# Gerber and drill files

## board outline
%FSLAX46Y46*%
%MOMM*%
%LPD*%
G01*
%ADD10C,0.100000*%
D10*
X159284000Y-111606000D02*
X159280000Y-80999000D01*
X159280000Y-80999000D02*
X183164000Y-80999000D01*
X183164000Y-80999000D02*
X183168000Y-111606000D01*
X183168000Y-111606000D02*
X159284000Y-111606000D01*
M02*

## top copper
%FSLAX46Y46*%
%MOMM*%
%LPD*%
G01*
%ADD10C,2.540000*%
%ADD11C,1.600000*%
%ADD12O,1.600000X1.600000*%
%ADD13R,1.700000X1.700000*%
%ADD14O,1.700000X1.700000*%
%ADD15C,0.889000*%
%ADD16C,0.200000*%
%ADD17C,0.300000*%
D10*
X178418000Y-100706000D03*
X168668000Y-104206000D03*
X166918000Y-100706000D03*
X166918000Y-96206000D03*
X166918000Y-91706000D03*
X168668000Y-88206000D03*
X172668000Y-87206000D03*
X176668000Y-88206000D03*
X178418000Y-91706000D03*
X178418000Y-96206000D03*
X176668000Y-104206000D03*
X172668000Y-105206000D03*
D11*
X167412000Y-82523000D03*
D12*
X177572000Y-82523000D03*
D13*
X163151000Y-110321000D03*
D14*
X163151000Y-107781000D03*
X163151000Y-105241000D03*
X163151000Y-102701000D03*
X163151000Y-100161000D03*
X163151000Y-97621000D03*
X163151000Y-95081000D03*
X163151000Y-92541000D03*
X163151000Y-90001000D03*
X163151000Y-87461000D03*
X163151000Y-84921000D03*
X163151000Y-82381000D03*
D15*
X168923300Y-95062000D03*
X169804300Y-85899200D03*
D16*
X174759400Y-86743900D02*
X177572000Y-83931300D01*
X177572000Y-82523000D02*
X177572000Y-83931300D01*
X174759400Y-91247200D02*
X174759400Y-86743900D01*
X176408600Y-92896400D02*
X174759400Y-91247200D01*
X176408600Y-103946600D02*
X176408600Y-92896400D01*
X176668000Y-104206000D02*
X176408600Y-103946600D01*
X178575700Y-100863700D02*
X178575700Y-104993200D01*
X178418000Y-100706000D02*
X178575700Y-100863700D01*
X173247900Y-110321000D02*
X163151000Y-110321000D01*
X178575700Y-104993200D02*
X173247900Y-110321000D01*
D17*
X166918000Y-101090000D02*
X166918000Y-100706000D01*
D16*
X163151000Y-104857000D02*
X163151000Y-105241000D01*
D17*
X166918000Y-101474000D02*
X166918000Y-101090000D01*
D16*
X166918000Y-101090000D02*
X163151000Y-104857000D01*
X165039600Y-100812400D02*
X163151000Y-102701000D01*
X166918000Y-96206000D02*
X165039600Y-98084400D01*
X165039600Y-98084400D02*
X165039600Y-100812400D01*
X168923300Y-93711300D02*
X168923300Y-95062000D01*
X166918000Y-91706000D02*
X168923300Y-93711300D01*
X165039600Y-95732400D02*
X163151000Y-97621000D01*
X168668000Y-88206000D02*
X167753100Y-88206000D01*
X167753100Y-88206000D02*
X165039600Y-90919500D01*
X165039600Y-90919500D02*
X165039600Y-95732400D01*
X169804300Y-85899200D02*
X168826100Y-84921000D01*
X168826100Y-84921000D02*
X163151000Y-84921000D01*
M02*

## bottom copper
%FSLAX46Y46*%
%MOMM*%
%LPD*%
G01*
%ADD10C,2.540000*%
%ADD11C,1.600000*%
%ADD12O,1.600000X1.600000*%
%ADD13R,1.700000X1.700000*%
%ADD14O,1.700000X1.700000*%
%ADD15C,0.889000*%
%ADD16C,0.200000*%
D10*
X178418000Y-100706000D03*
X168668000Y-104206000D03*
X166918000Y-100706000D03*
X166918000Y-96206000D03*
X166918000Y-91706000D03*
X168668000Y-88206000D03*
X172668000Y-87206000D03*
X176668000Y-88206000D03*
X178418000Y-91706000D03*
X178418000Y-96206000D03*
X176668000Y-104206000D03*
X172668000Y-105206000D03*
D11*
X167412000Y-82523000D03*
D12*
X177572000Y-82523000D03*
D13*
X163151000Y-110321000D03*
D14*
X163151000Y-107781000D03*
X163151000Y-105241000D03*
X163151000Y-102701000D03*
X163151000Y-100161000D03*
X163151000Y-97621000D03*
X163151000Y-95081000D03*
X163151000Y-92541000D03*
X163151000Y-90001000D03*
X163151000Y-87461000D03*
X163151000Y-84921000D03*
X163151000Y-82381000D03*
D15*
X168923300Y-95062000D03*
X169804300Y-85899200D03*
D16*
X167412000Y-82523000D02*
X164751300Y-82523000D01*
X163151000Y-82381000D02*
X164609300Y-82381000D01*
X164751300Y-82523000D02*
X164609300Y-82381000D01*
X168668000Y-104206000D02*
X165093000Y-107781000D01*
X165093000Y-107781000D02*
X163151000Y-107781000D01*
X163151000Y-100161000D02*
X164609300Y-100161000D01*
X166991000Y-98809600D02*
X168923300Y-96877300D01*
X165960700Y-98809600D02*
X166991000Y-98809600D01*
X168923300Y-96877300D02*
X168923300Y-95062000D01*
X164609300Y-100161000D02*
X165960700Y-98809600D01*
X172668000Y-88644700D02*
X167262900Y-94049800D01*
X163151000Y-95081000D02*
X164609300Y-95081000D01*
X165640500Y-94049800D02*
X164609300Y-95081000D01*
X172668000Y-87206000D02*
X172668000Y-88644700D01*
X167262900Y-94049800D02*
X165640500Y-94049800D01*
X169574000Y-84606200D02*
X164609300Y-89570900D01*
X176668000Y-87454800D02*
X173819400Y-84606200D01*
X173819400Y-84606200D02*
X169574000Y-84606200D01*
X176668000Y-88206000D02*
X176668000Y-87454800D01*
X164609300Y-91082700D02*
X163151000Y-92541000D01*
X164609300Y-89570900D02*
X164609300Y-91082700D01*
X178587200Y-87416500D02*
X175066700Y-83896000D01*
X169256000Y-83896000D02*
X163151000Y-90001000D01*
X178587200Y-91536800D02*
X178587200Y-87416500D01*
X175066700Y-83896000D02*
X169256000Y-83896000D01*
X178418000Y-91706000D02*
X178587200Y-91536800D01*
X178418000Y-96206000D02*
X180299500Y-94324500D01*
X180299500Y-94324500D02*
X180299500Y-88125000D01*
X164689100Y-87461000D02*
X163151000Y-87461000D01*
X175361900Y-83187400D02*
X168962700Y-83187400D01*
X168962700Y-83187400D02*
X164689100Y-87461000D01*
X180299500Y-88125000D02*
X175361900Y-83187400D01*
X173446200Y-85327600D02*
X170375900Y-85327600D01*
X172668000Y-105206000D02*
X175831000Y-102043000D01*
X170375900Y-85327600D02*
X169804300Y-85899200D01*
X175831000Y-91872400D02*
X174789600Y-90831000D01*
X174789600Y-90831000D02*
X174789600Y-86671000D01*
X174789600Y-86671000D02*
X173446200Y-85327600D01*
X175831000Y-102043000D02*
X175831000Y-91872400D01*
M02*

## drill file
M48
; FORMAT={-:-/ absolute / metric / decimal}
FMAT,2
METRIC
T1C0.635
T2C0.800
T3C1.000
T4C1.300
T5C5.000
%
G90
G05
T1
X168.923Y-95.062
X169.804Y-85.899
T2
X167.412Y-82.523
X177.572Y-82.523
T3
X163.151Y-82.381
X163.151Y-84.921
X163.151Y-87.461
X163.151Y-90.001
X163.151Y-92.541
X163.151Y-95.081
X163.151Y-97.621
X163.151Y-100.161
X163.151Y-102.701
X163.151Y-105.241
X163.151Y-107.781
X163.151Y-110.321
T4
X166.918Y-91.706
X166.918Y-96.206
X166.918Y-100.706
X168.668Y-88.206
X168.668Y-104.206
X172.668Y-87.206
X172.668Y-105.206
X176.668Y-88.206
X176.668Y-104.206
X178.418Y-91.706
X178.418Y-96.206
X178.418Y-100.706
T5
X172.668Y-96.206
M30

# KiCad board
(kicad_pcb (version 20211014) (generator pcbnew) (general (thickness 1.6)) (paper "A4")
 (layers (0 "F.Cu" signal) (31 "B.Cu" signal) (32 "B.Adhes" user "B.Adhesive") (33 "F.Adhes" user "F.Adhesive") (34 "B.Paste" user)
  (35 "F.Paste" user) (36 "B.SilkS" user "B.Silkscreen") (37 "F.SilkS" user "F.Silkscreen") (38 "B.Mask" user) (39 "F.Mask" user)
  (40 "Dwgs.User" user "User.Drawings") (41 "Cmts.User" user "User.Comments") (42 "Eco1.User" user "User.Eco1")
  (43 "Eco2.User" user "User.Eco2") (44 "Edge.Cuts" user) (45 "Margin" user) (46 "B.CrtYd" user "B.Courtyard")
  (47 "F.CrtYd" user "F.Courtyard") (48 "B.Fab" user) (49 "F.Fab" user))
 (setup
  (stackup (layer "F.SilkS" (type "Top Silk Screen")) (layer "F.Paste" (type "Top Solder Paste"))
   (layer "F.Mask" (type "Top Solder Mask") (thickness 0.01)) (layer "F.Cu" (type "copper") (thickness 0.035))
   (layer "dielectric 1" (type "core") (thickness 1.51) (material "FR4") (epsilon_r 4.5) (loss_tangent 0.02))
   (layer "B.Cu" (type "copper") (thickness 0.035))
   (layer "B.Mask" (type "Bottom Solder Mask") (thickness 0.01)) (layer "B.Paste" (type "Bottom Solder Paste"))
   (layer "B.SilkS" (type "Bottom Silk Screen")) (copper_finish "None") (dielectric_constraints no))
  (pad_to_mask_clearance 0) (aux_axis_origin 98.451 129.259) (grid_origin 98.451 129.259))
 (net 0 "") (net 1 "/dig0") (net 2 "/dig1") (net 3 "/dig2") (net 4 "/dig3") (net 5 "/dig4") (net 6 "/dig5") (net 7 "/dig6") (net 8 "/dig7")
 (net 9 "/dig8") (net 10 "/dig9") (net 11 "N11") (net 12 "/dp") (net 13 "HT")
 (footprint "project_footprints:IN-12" (layer "F.Cu") (at 172.668 96.206)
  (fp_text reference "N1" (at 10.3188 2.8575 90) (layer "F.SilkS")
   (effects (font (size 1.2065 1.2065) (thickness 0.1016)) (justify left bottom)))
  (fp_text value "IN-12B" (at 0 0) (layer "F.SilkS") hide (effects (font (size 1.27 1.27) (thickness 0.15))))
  (pad "" np_thru_hole circle locked (at 0 0) (size 5 5) (drill 5) (layers *.Cu *.Mask))
  (pad "0" thru_hole circle locked (at 5.75 4.5) (size 2.54 2.54) (drill 1.3) (layers *.Cu *.Mask) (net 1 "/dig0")
   (solder_mask_margin 0.1016))
  (pad "1" thru_hole circle locked (at -4 8) (size 2.54 2.54) (drill 1.3) (layers *.Cu *.Mask) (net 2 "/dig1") (solder_mask_margin 0.1016))
  (pad "2" thru_hole circle locked (at -5.75 4.5) (size 2.54 2.54) (drill 1.3) (layers *.Cu *.Mask) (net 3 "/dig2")
   (solder_mask_margin 0.1016))
  (pad "3" thru_hole circle locked (at -5.75 0) (size 2.54 2.54) (drill 1.3) (layers *.Cu *.Mask) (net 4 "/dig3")
   (solder_mask_margin 0.1016))
  (pad "4" thru_hole circle locked (at -5.75 -4.5) (size 2.54 2.54) (drill 1.3) (layers *.Cu *.Mask) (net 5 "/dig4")
   (solder_mask_margin 0.1016))
  (pad "5" thru_hole circle locked (at -4 -8) (size 2.54 2.54) (drill 1.3) (layers *.Cu *.Mask) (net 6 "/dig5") (solder_mask_margin 0.1016))
  (pad "6" thru_hole circle locked (at 0 -9) (size 2.54 2.54) (drill 1.3) (layers *.Cu *.Mask) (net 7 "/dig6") (solder_mask_margin 0.1016))
  (pad "7" thru_hole circle locked (at 4 -8) (size 2.54 2.54) (drill 1.3) (layers *.Cu *.Mask) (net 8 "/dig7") (solder_mask_margin 0.1016))
  (pad "8" thru_hole circle locked (at 5.75 -4.5) (size 2.54 2.54) (drill 1.3) (layers *.Cu *.Mask) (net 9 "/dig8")
   (solder_mask_margin 0.1016))
  (pad "9" thru_hole circle locked (at 5.75 0) (size 2.54 2.54) (drill 1.3) (layers *.Cu *.Mask) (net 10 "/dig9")
   (solder_mask_margin 0.1016))
  (pad "A" thru_hole circle locked (at 4 8) (size 2.54 2.54) (drill 1.3) (layers *.Cu *.Mask) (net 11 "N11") (solder_mask_margin 0.1016))
  (pad "LHDP" thru_hole circle locked (at 0 9) (size 2.54 2.54) (drill 1.3) (layers *.Cu *.Mask) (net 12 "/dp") (solder_mask_margin 0.1016)))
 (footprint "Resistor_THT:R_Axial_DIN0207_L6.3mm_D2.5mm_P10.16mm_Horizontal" (layer "F.Cu") (at 167.412 82.523)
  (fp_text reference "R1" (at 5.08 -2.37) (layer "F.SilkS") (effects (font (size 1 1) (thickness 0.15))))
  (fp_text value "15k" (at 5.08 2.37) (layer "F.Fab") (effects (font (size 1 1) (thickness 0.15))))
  (pad "1" thru_hole circle (at 0 0) (size 1.6 1.6) (drill 0.8) (layers *.Cu *.Mask) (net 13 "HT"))
  (pad "2" thru_hole oval (at 10.16 0) (size 1.6 1.6) (drill 0.8) (layers *.Cu *.Mask) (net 11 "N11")))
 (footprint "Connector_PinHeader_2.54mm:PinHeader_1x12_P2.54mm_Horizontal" (layer "F.Cu") (at 163.151 110.321 180)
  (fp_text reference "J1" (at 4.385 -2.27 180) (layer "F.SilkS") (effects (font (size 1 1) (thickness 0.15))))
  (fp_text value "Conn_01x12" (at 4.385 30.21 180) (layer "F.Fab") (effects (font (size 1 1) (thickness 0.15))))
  (pad "1" thru_hole rect (at 0 0 180) (size 1.7 1.7) (drill 1) (layers *.Cu *.Mask) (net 1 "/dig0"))
  (pad "2" thru_hole oval (at 0 2.54 180) (size 1.7 1.7) (drill 1) (layers *.Cu *.Mask) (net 2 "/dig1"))
  (pad "3" thru_hole oval (at 0 5.08 180) (size 1.7 1.7) (drill 1) (layers *.Cu *.Mask) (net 3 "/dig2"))
  (pad "4" thru_hole oval (at 0 7.62 180) (size 1.7 1.7) (drill 1) (layers *.Cu *.Mask) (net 4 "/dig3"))
  (pad "5" thru_hole oval (at 0 10.16 180) (size 1.7 1.7) (drill 1) (layers *.Cu *.Mask) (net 5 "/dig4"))
  (pad "6" thru_hole oval (at 0 12.7 180) (size 1.7 1.7) (drill 1) (layers *.Cu *.Mask) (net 6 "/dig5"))
  (pad "7" thru_hole oval (at 0 15.24 180) (size 1.7 1.7) (drill 1) (layers *.Cu *.Mask) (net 7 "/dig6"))
  (pad "8" thru_hole oval (at 0 17.78 180) (size 1.7 1.7) (drill 1) (layers *.Cu *.Mask) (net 8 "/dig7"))
  (pad "9" thru_hole oval (at 0 20.32 180) (size 1.7 1.7) (drill 1) (layers *.Cu *.Mask) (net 9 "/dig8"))
  (pad "10" thru_hole oval (at 0 22.86 180) (size 1.7 1.7) (drill 1) (layers *.Cu *.Mask) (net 10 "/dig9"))
  (pad "11" thru_hole oval (at 0 25.4 180) (size 1.7 1.7) (drill 1) (layers *.Cu *.Mask) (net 12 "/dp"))
  (pad "12" thru_hole oval (at 0 27.94 180) (size 1.7 1.7) (drill 1) (layers *.Cu *.Mask) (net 13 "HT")))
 (gr_line (start 159.284 111.606) (end 159.28 80.999) (layer "Edge.Cuts") (width 0.1))
 (gr_line (start 159.28 80.999) (end 183.164 80.999) (layer "Edge.Cuts") (width 0.1))
 (gr_line (start 183.164 80.999) (end 183.168 111.606) (layer "Edge.Cuts") (width 0.1))
 (gr_line (start 183.168 111.606) (end 159.284 111.606) (layer "Edge.Cuts") (width 0.1))
 (segment (start 174.7594 86.7439) (end 177.572 83.9313) (width 0.2) (layer "F.Cu") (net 11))
 (segment (start 177.572 82.523) (end 177.572 83.9313) (width 0.2) (layer "F.Cu") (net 11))
 (segment (start 174.7594 91.2472) (end 174.7594 86.7439) (width 0.2) (layer "F.Cu") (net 11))
 (segment (start 176.4086 92.8964) (end 174.7594 91.2472) (width 0.2) (layer "F.Cu") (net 11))
 (segment (start 176.4086 103.9466) (end 176.4086 92.8964) (width 0.2) (layer "F.Cu") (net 11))
 (segment (start 176.668 104.206) (end 176.4086 103.9466) (width 0.2) (layer "F.Cu") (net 11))
 (segment (start 178.5757 100.8637) (end 178.5757 104.9932) (width 0.2) (layer "F.Cu") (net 1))
 (segment (start 178.418 100.706) (end 178.5757 100.8637) (width 0.2) (layer "F.Cu") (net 1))
 (segment (start 173.2479 110.321) (end 163.151 110.321) (width 0.2) (layer "F.Cu") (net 1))
 (segment (start 178.5757 104.9932) (end 173.2479 110.321) (width 0.2) (layer "F.Cu") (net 1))
 (segment (start 167.412 82.523) (end 164.7513 82.523) (width 0.2) (layer "B.Cu") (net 13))
 (segment (start 163.151 82.381) (end 164.6093 82.381) (width 0.2) (layer "B.Cu") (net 13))
 (segment (start 164.7513 82.523) (end 164.6093 82.381) (width 0.2) (layer "B.Cu") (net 13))
 (segment (start 168.668 104.206) (end 165.093 107.781) (width 0.2) (layer "B.Cu") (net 2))
 (segment (start 165.093 107.781) (end 163.151 107.781) (width 0.2) (layer "B.Cu") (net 2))
 (segment (start 166.918 101.09) (end 166.918 100.706) (width 0.3) (layer "F.Cu") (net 3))
 (segment (start 163.151 104.857) (end 163.151 105.241) (width 0.2) (layer "F.Cu") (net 3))
 (segment (start 166.918 101.474) (end 166.918 101.09) (width 0.3) (layer "F.Cu") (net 3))
 (segment (start 166.918 101.09) (end 163.151 104.857) (width 0.2) (layer "F.Cu") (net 3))
 (segment (start 165.0396 100.8124) (end 163.151 102.701) (width 0.2) (layer "F.Cu") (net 4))
 (segment (start 166.918 96.206) (end 165.0396 98.0844) (width 0.2) (layer "F.Cu") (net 4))
 (segment (start 165.0396 98.0844) (end 165.0396 100.8124) (width 0.2) (layer "F.Cu") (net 4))
 (segment (start 168.9233 93.7113) (end 168.9233 95.062) (width 0.2) (layer "F.Cu") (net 5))
 (segment (start 166.918 91.706) (end 168.9233 93.7113) (width 0.2) (layer "F.Cu") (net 5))
 (via (at 168.9233 95.062) (size 0.889) (drill 0.635) (layers "F.Cu" "B.Cu") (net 5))
 (segment (start 163.151 100.161) (end 164.6093 100.161) (width 0.2) (layer "B.Cu") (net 5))
 (segment (start 166.991 98.8096) (end 168.9233 96.8773) (width 0.2) (layer "B.Cu") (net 5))
 (segment (start 165.9607 98.8096) (end 166.991 98.8096) (width 0.2) (layer "B.Cu") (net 5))
 (segment (start 168.9233 96.8773) (end 168.9233 95.062) (width 0.2) (layer "B.Cu") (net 5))
 (segment (start 164.6093 100.161) (end 165.9607 98.8096) (width 0.2) (layer "B.Cu") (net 5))
 (segment (start 165.0396 95.7324) (end 163.151 97.621) (width 0.2) (layer "F.Cu") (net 6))
 (segment (start 168.668 88.206) (end 167.7531 88.206) (width 0.2) (layer "F.Cu") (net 6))
 (segment (start 167.7531 88.206) (end 165.0396 90.9195) (width 0.2) (layer "F.Cu") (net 6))
 (segment (start 165.0396 90.9195) (end 165.0396 95.7324) (width 0.2) (layer "F.Cu") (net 6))
 (segment (start 172.668 88.6447) (end 167.2629 94.0498) (width 0.2) (layer "B.Cu") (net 7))
 (segment (start 163.151 95.081) (end 164.6093 95.081) (width 0.2) (layer "B.Cu") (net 7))
 (segment (start 165.6405 94.0498) (end 164.6093 95.081) (width 0.2) (layer "B.Cu") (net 7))
 (segment (start 172.668 87.206) (end 172.668 88.6447) (width 0.2) (layer "B.Cu") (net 7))
 (segment (start 167.2629 94.0498) (end 165.6405 94.0498) (width 0.2) (layer "B.Cu") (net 7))
 (segment (start 169.574 84.6062) (end 164.6093 89.5709) (width 0.2) (layer "B.Cu") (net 8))
 (segment (start 176.668 87.4548) (end 173.8194 84.6062) (width 0.2) (layer "B.Cu") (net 8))
 (segment (start 173.8194 84.6062) (end 169.574 84.6062) (width 0.2) (layer "B.Cu") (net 8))
 (segment (start 176.668 88.206) (end 176.668 87.4548) (width 0.2) (layer "B.Cu") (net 8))
 (segment (start 164.6093 91.0827) (end 163.151 92.541) (width 0.2) (layer "B.Cu") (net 8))
 (segment (start 164.6093 89.5709) (end 164.6093 91.0827) (width 0.2) (layer "B.Cu") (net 8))
 (segment (start 178.5872 87.4165) (end 175.0667 83.896) (width 0.2) (layer "B.Cu") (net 9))
 (segment (start 169.256 83.896) (end 163.151 90.001) (width 0.2) (layer "B.Cu") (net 9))
 (segment (start 178.5872 91.5368) (end 178.5872 87.4165) (width 0.2) (layer "B.Cu") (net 9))
 (segment (start 175.0667 83.896) (end 169.256 83.896) (width 0.2) (layer "B.Cu") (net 9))
 (segment (start 178.418 91.706) (end 178.5872 91.5368) (width 0.2) (layer "B.Cu") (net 9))
 (segment (start 178.418 96.206) (end 180.2995 94.3245) (width 0.2) (layer "B.Cu") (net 10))
 (segment (start 180.2995 94.3245) (end 180.2995 88.125) (width 0.2) (layer "B.Cu") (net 10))
 (segment (start 164.6891 87.461) (end 163.151 87.461) (width 0.2) (layer "B.Cu") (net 10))
 (segment (start 175.3619 83.1874) (end 168.9627 83.1874) (width 0.2) (layer "B.Cu") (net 10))
 (segment (start 168.9627 83.1874) (end 164.6891 87.461) (width 0.2) (layer "B.Cu") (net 10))
 (segment (start 180.2995 88.125) (end 175.3619 83.1874) (width 0.2) (layer "B.Cu") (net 10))
 (segment (start 169.8043 85.8992) (end 168.8261 84.921) (width 0.2) (layer "F.Cu") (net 12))
 (segment (start 168.8261 84.921) (end 163.151 84.921) (width 0.2) (layer "F.Cu") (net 12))
 (via (at 169.8043 85.8992) (size 0.889) (drill 0.635) (layers "F.Cu" "B.Cu") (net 12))
 (segment (start 173.4462 85.3276) (end 170.3759 85.3276) (width 0.2) (layer "B.Cu") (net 12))
 (segment (start 172.668 105.206) (end 175.831 102.043) (width 0.2) (layer "B.Cu") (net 12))
 (segment (start 170.3759 85.3276) (end 169.8043 85.8992) (width 0.2) (layer "B.Cu") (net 12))
 (segment (start 175.831 91.8724) (end 174.7896 90.831) (width 0.2) (layer "B.Cu") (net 12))
 (segment (start 174.7896 90.831) (end 174.7896 86.671) (width 0.2) (layer "B.Cu") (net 12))
 (segment (start 174.7896 86.671) (end 173.4462 85.3276) (width 0.2) (layer "B.Cu") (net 12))
 (segment (start 175.831 102.043) (end 175.831 91.8724) (width 0.2) (layer "B.Cu") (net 12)))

